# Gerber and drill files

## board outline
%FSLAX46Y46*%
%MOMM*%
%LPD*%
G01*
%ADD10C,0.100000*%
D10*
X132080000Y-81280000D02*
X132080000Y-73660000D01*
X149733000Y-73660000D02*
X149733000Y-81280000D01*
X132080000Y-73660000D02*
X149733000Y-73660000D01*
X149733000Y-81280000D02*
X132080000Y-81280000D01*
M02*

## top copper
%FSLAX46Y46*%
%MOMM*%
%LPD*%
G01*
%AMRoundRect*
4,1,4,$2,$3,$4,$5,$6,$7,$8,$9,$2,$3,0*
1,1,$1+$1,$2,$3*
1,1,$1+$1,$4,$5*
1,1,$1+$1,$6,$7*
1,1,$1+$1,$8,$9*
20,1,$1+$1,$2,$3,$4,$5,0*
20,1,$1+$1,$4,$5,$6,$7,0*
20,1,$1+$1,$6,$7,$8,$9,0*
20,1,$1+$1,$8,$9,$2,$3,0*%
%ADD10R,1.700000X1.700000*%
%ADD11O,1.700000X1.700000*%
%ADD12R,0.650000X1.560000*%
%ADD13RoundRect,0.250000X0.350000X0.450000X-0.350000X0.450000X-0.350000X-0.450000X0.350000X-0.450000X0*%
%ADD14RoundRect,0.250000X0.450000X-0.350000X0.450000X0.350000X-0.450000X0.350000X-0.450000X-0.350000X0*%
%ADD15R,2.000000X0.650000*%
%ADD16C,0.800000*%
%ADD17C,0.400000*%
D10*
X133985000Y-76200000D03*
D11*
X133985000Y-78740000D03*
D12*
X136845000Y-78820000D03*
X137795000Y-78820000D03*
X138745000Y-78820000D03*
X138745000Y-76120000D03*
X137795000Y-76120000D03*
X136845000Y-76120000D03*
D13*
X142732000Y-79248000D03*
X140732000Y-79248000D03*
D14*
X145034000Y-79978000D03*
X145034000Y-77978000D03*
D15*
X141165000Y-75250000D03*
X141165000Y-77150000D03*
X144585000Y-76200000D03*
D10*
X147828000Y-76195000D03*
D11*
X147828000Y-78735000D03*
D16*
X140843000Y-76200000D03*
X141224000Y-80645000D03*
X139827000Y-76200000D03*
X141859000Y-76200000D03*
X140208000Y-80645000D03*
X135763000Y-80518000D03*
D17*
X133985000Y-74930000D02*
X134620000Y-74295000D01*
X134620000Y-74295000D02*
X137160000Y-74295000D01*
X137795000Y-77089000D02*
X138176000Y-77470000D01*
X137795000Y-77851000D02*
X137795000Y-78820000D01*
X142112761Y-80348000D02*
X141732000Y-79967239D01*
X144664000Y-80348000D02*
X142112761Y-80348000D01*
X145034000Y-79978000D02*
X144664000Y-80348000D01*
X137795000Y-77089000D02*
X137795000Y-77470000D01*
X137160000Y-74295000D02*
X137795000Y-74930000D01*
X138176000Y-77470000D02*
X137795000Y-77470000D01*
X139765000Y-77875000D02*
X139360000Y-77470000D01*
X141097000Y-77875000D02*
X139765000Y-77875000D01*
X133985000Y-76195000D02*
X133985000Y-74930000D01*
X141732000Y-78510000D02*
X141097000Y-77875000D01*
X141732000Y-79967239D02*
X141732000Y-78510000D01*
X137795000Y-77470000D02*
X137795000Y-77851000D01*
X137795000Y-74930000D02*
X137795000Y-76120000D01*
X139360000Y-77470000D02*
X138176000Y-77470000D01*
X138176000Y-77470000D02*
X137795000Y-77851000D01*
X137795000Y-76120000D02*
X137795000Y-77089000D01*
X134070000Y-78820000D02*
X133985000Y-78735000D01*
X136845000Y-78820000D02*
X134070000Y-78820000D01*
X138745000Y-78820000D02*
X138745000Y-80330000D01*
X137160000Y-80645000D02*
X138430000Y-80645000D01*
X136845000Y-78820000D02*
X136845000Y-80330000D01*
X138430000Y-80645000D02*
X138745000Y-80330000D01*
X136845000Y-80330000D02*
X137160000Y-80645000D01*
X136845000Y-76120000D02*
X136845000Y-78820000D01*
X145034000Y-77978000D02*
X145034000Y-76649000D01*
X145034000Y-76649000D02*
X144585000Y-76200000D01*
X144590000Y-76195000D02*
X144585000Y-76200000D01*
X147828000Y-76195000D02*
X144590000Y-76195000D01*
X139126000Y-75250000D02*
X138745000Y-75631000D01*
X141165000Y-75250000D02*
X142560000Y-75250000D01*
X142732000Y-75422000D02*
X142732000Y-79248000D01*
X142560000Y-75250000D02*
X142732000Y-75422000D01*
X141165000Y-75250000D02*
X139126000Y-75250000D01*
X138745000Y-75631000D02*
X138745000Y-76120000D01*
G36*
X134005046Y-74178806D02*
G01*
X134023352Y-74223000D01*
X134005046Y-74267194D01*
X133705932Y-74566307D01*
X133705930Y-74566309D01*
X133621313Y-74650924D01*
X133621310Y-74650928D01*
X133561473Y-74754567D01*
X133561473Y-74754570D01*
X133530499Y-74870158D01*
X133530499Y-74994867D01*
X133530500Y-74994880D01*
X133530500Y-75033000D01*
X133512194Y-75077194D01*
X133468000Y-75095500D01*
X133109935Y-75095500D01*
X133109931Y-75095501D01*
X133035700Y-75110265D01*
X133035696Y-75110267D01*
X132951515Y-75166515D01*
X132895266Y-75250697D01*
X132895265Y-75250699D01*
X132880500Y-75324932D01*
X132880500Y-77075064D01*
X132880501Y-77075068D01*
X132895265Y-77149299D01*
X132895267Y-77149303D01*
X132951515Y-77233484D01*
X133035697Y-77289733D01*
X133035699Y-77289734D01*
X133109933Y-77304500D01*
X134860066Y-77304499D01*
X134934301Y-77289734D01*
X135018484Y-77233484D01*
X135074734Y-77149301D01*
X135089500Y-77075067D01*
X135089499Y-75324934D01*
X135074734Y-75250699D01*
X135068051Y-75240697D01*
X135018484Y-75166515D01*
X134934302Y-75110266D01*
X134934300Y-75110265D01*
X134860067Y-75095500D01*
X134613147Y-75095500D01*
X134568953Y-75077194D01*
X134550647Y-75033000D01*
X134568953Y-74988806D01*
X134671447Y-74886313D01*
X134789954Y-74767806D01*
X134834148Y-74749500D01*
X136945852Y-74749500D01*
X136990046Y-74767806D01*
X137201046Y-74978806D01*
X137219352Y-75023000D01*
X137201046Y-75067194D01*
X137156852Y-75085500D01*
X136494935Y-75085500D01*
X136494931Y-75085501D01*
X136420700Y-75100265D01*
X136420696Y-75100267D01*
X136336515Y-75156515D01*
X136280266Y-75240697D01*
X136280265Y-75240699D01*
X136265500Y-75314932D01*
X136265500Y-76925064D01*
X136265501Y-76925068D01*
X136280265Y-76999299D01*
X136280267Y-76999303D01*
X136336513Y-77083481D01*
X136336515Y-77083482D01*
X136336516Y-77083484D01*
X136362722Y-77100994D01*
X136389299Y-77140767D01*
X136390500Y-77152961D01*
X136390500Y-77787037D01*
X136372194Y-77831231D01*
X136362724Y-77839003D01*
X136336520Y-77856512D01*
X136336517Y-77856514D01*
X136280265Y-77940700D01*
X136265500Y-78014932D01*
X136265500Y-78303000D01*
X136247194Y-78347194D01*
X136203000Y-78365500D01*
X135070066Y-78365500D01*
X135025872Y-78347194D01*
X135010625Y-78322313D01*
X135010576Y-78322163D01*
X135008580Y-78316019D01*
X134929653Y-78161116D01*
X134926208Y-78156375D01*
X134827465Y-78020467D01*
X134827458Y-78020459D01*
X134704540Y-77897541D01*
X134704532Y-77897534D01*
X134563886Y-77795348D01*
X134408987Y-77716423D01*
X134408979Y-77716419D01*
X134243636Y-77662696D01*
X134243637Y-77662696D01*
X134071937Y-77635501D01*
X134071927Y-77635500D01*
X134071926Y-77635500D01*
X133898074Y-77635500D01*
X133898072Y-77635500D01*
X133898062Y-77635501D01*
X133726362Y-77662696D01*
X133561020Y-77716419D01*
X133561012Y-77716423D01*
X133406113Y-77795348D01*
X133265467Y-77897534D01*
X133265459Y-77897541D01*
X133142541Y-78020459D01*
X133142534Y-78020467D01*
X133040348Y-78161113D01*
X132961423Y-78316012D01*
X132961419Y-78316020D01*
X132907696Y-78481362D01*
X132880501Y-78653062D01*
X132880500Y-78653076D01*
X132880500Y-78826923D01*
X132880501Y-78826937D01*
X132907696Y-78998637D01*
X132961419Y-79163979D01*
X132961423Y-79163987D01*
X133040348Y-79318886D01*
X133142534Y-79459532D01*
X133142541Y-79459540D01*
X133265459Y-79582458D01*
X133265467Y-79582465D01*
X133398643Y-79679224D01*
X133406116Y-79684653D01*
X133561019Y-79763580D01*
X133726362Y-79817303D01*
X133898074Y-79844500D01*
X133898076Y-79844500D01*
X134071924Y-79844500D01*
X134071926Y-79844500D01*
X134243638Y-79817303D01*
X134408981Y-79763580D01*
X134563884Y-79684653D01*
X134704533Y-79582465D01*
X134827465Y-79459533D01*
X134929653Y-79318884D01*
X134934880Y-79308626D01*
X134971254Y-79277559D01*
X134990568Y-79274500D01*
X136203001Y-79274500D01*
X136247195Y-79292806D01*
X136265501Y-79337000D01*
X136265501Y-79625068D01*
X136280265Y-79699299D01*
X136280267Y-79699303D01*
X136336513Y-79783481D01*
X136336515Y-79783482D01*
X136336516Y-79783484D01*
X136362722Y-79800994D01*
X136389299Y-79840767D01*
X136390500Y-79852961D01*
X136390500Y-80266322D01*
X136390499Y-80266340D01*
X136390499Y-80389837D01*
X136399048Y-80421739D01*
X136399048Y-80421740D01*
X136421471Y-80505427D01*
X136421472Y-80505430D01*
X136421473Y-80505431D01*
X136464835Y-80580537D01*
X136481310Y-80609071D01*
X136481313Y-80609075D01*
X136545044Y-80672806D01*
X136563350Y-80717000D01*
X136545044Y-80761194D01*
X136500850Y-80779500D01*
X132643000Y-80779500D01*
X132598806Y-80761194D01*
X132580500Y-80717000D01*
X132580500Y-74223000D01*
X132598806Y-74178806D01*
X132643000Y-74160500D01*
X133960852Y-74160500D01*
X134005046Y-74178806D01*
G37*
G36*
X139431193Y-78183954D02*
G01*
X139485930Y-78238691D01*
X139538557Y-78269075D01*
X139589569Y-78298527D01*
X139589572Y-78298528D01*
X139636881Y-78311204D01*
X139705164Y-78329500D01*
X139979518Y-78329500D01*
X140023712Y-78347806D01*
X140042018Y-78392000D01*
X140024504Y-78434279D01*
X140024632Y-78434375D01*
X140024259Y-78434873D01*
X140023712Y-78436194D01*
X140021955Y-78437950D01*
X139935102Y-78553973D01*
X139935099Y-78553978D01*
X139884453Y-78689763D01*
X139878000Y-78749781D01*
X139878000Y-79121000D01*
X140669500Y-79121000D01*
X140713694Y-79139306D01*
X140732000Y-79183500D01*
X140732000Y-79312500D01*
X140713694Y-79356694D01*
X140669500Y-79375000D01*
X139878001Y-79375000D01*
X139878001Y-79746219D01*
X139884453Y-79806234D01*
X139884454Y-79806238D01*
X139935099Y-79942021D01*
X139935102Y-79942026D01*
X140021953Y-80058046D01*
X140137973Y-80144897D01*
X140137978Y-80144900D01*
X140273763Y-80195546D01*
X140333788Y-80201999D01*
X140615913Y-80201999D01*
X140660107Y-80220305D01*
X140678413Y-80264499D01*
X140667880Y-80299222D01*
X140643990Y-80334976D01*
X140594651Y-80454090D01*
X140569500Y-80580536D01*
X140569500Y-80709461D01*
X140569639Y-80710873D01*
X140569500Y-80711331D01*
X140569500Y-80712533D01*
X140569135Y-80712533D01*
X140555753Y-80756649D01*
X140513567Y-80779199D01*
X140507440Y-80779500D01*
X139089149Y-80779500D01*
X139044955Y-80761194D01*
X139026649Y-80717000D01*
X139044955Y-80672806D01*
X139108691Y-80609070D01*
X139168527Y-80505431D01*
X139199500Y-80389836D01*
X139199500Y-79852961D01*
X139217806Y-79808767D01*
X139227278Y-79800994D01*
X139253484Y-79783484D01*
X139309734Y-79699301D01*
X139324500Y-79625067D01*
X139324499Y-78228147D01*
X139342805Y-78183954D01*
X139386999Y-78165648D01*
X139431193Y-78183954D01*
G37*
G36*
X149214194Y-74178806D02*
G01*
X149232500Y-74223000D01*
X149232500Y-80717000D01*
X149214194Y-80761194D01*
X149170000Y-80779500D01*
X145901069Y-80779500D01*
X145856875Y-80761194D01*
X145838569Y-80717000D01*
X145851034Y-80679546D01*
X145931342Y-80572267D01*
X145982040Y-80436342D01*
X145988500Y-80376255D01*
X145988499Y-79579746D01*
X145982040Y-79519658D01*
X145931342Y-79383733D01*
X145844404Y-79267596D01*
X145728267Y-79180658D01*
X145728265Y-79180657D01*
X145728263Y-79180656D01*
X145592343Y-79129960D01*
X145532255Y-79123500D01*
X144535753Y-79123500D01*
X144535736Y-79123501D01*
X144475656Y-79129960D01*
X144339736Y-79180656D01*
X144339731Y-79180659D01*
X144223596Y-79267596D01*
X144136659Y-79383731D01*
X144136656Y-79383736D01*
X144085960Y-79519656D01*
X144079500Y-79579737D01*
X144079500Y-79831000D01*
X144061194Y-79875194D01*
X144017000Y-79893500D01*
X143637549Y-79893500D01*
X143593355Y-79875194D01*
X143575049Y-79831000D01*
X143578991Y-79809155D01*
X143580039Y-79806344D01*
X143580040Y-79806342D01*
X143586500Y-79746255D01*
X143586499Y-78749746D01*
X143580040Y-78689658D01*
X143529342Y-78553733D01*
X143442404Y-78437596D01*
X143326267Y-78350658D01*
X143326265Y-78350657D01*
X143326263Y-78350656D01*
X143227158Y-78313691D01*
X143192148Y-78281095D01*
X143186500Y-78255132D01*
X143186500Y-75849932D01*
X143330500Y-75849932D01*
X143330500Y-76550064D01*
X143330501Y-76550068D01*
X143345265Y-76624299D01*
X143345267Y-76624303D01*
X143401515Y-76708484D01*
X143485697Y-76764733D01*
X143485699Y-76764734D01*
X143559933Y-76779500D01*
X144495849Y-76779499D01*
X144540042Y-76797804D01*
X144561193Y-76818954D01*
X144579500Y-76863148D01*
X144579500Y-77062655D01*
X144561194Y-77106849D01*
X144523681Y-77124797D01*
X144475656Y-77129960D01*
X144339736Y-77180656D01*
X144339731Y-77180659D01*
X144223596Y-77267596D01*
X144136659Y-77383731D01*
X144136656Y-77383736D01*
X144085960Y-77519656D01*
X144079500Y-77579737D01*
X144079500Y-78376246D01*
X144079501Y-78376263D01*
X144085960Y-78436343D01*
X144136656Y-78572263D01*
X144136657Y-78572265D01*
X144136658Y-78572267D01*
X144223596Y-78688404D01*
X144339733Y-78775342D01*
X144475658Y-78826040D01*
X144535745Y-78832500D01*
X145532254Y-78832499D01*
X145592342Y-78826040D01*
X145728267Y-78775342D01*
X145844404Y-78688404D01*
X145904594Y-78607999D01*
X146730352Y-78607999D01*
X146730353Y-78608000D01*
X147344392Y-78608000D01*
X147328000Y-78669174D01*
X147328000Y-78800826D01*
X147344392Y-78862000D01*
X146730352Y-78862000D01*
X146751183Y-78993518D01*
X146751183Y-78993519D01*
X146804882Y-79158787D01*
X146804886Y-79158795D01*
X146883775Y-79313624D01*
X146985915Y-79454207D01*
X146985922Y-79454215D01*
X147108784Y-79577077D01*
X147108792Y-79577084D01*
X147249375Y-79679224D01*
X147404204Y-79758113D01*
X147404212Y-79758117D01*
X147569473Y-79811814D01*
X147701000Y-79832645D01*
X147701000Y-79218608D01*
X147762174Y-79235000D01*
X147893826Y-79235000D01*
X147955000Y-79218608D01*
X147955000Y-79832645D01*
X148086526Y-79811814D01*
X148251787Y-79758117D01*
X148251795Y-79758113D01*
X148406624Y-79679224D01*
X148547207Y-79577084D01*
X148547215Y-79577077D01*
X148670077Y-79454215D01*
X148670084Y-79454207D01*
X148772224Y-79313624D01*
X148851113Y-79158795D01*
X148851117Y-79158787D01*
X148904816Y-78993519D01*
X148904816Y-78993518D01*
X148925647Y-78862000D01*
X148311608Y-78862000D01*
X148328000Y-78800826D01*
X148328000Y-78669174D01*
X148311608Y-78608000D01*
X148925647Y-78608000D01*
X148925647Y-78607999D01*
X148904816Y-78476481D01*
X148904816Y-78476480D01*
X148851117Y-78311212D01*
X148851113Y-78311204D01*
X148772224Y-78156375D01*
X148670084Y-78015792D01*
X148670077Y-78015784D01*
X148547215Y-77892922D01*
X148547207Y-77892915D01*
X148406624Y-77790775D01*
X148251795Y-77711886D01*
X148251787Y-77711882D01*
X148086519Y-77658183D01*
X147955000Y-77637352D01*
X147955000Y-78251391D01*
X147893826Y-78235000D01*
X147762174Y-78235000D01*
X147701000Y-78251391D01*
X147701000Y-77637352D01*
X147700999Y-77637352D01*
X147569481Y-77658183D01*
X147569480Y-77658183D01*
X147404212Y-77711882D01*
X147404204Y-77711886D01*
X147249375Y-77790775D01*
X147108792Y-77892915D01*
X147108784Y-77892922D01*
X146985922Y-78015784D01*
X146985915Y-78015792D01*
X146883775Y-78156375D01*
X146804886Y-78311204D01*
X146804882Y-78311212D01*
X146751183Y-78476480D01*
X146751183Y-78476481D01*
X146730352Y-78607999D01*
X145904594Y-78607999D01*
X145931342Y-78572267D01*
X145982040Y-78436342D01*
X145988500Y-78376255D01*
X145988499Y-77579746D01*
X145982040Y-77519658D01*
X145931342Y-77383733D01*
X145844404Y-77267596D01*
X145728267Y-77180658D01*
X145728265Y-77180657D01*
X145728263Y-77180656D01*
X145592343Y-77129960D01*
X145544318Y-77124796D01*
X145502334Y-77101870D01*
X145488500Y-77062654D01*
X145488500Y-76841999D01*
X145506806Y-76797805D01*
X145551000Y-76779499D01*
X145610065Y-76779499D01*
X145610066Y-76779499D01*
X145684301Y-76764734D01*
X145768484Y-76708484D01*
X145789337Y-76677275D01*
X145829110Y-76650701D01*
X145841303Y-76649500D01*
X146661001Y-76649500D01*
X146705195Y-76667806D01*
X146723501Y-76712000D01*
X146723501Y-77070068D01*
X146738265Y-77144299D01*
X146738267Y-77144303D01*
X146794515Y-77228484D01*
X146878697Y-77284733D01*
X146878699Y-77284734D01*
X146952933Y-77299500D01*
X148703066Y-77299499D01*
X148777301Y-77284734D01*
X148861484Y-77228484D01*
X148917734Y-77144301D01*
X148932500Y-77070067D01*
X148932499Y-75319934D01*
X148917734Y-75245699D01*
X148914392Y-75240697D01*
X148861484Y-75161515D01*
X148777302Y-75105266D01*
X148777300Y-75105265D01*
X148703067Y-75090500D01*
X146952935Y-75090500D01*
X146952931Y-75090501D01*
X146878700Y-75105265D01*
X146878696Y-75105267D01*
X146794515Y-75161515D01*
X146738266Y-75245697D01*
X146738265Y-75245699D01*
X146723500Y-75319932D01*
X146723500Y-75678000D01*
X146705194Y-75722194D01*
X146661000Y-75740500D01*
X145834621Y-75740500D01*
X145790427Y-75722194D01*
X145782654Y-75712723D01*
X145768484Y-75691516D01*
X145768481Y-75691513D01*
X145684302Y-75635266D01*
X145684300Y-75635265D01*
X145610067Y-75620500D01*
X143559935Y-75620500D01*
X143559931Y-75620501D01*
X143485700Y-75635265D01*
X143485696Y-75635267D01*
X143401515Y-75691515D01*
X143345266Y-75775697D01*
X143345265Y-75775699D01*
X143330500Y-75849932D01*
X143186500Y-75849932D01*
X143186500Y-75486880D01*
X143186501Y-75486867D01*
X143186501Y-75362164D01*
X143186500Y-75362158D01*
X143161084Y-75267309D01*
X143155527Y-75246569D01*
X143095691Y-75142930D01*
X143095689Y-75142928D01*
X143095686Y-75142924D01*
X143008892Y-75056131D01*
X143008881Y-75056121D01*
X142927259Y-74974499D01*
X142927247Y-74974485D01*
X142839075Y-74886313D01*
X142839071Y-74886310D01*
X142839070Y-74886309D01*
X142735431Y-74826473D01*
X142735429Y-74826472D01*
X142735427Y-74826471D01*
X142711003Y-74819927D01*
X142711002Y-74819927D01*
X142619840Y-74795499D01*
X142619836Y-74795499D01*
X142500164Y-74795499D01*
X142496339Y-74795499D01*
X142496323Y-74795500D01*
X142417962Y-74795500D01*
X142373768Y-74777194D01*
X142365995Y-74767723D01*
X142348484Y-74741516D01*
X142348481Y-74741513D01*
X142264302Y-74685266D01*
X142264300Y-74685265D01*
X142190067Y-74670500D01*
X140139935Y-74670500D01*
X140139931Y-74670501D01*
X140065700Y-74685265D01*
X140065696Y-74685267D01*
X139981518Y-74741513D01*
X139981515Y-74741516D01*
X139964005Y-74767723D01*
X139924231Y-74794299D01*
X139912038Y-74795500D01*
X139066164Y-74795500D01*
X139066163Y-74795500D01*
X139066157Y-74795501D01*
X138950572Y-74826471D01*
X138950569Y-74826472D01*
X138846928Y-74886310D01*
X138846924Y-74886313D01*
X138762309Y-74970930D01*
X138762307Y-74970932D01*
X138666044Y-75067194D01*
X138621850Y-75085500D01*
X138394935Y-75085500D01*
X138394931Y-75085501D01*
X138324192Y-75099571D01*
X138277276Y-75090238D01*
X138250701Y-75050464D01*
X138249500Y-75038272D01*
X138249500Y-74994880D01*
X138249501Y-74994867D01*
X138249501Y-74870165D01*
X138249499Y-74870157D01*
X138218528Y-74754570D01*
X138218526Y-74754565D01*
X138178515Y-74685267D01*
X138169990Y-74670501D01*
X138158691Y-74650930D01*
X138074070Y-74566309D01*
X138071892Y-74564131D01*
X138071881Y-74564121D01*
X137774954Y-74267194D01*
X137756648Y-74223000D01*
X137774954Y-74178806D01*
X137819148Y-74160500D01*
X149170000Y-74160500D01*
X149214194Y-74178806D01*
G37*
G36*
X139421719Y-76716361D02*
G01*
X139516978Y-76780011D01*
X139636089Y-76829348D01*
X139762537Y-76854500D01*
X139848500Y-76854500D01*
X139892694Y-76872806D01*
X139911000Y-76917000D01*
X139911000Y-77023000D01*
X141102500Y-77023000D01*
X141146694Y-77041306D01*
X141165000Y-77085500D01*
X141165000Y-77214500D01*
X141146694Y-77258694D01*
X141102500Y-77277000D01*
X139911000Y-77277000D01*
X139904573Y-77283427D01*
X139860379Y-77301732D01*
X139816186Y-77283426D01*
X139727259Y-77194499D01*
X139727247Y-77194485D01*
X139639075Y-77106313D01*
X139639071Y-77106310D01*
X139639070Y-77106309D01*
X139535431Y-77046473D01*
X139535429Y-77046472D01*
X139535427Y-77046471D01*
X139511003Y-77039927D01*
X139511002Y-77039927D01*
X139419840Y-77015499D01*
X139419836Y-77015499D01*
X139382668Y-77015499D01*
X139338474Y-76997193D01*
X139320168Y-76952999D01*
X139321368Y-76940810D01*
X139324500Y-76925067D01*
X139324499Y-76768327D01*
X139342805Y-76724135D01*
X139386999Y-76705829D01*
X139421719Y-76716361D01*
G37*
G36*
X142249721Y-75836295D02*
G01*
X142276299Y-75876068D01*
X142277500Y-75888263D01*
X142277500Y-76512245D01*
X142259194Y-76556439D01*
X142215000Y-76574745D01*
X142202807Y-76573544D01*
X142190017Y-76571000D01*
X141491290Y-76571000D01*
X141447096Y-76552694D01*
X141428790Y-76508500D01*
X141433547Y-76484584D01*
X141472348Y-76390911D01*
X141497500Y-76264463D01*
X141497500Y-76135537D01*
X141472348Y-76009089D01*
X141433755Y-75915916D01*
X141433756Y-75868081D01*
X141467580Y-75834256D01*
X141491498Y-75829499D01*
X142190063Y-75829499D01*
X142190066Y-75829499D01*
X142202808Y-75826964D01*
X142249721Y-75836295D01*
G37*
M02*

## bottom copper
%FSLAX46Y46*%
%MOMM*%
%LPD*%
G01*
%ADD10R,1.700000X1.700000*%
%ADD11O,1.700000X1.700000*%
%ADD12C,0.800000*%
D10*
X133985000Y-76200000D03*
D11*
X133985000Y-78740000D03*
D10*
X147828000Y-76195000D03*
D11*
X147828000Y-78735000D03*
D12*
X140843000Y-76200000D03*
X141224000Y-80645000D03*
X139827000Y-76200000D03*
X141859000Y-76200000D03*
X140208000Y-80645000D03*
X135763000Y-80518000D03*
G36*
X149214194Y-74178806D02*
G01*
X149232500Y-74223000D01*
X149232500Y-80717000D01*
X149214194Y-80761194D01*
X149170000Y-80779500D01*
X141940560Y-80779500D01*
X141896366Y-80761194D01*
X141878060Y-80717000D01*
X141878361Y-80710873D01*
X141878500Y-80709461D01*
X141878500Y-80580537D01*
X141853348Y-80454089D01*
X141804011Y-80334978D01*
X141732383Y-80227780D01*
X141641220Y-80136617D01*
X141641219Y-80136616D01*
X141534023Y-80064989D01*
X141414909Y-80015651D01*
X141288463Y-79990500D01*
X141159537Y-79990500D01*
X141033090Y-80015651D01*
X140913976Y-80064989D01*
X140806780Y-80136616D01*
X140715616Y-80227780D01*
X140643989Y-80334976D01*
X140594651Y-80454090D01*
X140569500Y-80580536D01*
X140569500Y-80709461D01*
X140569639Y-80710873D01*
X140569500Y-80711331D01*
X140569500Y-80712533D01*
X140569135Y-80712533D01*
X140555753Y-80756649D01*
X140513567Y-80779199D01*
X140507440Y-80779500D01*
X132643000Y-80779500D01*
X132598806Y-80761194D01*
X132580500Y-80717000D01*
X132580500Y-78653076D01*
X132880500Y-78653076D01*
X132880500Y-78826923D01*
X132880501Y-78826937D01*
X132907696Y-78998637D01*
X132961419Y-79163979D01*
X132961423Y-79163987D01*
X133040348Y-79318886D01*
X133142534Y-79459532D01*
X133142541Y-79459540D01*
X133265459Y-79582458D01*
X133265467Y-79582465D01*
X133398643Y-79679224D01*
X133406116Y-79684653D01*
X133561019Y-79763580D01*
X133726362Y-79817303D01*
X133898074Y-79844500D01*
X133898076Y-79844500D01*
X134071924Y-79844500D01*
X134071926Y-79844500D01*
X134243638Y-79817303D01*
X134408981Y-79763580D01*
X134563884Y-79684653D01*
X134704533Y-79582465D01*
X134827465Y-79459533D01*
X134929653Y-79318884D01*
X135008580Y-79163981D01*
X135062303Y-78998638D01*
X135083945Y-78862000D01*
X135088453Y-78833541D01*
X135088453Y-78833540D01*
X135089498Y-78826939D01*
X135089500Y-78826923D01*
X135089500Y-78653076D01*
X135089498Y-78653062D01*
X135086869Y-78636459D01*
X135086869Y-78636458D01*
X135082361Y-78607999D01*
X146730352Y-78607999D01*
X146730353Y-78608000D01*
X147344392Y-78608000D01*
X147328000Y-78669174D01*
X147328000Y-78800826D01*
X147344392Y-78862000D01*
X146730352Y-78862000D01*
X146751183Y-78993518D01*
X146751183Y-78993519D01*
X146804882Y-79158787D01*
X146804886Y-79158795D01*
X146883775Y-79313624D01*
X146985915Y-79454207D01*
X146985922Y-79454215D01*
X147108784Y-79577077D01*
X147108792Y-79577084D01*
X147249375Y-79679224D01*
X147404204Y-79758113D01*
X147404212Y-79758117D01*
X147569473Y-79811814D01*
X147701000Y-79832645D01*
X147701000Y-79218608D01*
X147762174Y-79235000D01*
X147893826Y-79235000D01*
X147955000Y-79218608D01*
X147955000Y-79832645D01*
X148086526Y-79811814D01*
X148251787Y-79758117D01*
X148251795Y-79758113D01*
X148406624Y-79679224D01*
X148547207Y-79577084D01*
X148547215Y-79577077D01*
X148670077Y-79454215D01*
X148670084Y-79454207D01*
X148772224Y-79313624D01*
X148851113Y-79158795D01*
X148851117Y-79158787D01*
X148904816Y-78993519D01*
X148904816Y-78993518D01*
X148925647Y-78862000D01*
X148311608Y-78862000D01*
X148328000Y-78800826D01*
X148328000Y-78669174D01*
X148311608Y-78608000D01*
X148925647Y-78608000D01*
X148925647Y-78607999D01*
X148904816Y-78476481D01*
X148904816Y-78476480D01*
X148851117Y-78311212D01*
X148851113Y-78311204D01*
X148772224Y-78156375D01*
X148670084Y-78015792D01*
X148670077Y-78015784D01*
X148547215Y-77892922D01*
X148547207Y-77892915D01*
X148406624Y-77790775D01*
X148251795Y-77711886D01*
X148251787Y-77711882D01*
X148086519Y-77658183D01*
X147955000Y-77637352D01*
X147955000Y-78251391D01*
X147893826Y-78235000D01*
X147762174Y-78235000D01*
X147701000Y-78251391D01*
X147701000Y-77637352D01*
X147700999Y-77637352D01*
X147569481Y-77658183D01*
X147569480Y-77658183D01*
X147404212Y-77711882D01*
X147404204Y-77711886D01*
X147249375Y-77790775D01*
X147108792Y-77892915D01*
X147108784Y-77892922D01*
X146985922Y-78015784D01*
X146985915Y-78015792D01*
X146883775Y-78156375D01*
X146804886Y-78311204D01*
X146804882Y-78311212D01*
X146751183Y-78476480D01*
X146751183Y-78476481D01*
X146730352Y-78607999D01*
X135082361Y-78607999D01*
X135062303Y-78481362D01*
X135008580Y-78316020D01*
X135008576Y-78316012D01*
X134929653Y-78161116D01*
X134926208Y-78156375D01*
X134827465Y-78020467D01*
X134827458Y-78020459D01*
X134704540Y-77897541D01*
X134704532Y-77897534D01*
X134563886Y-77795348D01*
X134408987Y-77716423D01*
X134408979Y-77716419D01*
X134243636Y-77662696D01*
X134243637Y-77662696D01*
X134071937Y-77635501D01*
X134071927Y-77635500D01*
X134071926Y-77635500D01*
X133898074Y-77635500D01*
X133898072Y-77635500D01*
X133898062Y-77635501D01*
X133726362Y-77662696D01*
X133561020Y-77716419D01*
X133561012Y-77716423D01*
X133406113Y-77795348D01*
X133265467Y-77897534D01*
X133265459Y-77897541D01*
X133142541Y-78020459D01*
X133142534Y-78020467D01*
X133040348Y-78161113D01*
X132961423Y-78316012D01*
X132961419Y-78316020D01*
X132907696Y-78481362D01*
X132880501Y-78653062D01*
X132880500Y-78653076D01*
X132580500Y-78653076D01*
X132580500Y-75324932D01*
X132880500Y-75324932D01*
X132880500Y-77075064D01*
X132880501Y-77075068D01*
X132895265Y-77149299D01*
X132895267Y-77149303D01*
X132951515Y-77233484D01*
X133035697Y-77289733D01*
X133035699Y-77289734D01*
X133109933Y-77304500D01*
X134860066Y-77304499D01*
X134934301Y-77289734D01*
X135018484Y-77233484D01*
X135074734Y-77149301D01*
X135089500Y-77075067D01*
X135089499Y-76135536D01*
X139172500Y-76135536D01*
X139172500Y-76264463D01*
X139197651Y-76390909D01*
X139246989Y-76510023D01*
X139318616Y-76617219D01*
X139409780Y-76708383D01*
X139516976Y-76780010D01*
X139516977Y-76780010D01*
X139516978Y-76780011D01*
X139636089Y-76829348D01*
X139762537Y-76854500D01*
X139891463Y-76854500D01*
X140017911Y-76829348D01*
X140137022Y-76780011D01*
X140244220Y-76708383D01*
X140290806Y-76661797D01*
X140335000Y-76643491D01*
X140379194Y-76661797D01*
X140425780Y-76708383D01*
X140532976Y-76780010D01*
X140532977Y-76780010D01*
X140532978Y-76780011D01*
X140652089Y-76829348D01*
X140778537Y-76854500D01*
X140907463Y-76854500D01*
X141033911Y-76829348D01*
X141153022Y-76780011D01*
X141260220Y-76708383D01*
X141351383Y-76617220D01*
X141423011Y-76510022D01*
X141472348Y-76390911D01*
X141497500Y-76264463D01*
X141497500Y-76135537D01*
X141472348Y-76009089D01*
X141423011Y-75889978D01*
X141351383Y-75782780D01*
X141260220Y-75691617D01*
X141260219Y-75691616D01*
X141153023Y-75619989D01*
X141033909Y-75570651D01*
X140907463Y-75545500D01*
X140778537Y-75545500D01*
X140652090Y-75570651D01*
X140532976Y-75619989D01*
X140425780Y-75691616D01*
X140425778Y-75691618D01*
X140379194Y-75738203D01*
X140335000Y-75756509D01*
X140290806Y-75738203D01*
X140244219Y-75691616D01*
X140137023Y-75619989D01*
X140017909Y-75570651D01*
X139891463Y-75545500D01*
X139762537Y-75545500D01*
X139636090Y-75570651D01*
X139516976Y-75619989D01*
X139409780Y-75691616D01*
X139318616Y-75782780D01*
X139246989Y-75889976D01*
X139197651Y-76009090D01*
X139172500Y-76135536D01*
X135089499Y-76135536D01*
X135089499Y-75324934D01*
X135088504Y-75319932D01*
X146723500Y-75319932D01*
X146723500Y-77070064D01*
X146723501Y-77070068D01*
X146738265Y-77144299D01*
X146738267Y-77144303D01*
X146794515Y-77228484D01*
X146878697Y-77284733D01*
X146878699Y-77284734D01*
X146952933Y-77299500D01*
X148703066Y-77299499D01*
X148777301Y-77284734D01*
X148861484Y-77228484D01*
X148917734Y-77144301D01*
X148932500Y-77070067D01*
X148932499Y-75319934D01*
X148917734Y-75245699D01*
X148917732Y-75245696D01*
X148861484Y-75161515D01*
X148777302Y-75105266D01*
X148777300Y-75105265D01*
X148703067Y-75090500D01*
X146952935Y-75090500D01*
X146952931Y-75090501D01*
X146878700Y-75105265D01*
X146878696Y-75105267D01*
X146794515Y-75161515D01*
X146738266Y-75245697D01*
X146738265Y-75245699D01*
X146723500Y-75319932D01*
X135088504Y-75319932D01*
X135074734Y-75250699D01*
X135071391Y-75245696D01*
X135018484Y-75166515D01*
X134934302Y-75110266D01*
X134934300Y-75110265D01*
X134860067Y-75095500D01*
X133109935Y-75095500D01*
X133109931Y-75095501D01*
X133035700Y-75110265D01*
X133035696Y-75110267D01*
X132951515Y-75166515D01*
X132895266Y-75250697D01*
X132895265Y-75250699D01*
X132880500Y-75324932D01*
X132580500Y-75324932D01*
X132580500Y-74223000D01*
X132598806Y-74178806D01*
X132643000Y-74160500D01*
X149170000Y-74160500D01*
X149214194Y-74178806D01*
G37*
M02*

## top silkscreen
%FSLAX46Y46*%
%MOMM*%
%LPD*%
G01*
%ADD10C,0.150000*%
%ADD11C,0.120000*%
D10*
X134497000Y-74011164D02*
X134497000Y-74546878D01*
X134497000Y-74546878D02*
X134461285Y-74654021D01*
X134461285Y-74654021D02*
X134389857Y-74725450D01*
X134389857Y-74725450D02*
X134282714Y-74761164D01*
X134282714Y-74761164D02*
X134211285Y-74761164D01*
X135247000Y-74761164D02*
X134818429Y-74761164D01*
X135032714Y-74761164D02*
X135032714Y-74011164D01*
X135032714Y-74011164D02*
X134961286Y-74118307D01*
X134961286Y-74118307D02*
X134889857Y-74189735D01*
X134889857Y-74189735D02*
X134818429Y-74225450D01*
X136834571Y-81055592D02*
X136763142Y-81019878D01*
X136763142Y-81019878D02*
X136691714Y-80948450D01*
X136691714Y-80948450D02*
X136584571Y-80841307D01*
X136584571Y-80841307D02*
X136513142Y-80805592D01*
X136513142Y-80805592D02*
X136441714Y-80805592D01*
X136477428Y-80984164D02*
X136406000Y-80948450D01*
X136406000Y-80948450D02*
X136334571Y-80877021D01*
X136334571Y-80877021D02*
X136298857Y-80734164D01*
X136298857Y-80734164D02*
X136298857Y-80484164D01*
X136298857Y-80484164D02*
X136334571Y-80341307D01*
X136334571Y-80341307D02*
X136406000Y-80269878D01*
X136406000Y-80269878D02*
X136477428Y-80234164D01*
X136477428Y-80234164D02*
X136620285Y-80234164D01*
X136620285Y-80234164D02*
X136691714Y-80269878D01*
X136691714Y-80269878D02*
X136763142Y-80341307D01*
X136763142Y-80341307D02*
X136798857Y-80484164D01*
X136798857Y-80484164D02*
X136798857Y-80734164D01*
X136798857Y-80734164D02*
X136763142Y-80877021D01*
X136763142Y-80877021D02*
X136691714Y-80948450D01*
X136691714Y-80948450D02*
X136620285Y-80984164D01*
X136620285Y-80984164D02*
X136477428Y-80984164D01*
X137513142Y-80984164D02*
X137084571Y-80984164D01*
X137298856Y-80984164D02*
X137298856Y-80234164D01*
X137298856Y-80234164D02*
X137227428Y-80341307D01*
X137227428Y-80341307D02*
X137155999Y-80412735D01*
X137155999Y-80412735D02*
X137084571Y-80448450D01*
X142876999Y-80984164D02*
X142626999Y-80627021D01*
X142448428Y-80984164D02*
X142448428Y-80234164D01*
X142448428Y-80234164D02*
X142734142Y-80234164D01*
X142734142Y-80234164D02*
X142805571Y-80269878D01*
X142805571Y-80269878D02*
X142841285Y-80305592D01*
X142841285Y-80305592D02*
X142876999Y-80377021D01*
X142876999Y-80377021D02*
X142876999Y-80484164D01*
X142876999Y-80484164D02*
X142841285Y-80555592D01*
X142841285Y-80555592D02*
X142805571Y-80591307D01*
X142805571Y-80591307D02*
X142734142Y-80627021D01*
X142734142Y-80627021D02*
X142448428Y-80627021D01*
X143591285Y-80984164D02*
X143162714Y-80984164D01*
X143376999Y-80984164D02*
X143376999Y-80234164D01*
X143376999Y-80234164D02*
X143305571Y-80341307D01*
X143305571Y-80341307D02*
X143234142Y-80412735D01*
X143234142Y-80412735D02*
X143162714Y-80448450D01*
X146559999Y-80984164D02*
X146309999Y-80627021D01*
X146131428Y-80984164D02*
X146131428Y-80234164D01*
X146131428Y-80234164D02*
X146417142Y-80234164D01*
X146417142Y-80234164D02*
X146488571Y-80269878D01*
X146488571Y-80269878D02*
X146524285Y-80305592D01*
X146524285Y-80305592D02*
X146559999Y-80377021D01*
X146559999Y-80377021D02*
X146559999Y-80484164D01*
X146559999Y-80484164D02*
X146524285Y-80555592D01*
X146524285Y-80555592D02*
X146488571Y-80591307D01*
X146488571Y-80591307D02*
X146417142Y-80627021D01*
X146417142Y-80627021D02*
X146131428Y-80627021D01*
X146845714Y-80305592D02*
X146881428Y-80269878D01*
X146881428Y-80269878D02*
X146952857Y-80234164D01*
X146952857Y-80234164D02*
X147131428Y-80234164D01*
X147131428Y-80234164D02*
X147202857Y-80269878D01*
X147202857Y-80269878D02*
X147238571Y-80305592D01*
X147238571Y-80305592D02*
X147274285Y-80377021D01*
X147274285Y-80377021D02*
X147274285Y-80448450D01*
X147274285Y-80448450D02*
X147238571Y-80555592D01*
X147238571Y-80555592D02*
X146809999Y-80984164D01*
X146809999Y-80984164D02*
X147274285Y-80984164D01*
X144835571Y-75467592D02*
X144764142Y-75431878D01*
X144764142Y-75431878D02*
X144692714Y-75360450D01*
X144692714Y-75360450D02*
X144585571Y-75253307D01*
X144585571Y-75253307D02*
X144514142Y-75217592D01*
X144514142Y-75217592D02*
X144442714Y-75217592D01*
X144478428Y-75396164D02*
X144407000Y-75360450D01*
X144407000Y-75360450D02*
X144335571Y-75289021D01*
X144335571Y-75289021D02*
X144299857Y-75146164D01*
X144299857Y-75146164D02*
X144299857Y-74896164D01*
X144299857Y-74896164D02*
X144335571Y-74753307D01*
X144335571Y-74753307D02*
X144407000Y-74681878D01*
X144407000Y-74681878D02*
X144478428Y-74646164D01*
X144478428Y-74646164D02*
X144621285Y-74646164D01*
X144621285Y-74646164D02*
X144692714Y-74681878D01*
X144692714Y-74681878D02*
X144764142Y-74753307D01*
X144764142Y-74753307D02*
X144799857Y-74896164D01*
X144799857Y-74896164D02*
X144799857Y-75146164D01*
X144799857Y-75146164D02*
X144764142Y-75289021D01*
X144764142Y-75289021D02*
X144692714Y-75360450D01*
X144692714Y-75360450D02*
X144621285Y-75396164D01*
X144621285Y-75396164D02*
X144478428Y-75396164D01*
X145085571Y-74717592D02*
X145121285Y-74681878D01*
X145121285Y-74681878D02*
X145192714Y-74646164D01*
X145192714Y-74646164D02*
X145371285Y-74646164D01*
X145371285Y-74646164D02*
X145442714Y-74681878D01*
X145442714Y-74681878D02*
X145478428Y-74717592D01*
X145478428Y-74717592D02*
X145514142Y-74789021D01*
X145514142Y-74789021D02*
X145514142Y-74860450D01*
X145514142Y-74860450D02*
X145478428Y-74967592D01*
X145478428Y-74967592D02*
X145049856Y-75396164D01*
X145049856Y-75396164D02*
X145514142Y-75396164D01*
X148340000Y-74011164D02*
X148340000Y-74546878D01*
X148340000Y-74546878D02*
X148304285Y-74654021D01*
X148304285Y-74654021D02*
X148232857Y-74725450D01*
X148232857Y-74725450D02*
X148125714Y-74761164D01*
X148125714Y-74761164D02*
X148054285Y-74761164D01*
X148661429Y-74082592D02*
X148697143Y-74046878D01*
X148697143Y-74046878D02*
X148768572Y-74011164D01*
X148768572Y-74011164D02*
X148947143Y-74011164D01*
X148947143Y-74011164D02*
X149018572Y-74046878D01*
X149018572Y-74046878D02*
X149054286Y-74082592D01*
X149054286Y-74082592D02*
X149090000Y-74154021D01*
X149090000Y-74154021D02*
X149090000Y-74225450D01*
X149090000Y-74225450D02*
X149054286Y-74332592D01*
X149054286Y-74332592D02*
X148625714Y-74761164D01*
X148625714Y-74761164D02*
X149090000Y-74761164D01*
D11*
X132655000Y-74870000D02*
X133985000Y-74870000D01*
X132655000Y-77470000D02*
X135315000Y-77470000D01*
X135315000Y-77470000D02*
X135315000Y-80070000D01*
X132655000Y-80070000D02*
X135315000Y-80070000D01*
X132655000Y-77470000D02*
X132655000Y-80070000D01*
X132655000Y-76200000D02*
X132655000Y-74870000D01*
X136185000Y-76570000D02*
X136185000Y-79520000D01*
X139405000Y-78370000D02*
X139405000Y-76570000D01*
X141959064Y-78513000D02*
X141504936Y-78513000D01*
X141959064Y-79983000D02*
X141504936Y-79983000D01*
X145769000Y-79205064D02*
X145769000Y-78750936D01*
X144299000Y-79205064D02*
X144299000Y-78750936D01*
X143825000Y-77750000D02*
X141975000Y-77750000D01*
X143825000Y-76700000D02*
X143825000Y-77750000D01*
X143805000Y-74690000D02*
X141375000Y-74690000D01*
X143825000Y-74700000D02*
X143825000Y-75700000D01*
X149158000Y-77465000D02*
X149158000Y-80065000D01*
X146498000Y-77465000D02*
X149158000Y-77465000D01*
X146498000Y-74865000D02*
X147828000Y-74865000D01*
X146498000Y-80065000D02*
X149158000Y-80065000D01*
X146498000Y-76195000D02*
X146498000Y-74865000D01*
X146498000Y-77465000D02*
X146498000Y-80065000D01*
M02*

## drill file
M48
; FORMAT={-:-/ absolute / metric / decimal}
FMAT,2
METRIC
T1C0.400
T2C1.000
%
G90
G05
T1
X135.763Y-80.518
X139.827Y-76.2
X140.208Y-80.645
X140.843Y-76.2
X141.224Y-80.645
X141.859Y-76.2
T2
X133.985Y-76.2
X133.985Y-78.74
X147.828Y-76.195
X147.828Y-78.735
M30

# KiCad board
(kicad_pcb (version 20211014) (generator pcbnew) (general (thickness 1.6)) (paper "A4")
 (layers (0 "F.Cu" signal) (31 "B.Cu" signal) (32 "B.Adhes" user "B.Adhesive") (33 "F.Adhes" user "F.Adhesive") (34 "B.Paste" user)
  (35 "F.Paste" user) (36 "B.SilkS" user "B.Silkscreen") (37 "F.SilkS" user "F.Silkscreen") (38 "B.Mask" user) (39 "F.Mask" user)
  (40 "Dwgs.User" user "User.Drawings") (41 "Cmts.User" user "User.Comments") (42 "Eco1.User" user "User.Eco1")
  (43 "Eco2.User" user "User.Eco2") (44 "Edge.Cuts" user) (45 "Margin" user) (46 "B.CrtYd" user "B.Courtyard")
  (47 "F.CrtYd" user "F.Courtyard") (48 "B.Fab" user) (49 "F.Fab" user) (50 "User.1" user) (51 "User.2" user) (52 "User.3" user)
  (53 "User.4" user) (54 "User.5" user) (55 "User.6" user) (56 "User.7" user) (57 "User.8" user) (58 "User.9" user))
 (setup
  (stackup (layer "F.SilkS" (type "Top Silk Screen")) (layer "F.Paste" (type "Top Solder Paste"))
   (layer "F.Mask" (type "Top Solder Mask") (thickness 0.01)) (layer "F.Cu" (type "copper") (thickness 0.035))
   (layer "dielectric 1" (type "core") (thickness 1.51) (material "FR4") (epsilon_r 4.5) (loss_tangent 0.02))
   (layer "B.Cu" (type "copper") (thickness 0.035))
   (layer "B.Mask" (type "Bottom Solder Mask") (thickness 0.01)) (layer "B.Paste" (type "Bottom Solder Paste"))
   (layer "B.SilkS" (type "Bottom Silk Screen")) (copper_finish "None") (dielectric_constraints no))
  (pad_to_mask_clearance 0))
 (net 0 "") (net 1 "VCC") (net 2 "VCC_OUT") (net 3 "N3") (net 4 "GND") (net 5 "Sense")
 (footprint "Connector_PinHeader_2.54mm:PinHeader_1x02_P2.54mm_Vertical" (layer "F.Cu") (at 133.985 76.2)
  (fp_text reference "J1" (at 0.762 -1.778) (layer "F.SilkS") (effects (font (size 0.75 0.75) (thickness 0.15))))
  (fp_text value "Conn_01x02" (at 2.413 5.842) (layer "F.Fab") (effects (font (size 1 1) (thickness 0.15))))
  (fp_line (start -1.33 -1.33) (end 0 -1.33) (layer "F.SilkS") (width 0.12))
  (fp_line (start -1.33 1.27) (end 1.33 1.27) (layer "F.SilkS") (width 0.12))
  (fp_line (start 1.33 1.27) (end 1.33 3.87) (layer "F.SilkS") (width 0.12))
  (fp_line (start -1.33 3.87) (end 1.33 3.87) (layer "F.SilkS") (width 0.12))
  (fp_line (start -1.33 1.27) (end -1.33 3.87) (layer "F.SilkS") (width 0.12))
  (fp_line (start -1.33 0) (end -1.33 -1.33) (layer "F.SilkS") (width 0.12))
  (pad "1" thru_hole rect (at 0 0) (size 1.7 1.7) (drill 1) (layers *.Cu *.Mask) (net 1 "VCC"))
  (pad "2" thru_hole oval (at 0 2.54) (size 1.7 1.7) (drill 1) (layers *.Cu *.Mask) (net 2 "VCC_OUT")))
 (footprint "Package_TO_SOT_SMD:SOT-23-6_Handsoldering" (layer "F.Cu") (at 137.795 77.47 90)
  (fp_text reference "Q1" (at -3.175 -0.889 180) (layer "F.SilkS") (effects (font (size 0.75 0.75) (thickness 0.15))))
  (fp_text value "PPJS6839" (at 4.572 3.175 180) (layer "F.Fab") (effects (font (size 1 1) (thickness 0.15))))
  (fp_line (start 0.9 -1.61) (end -2.05 -1.61) (layer "F.SilkS") (width 0.12))
  (fp_line (start -0.9 1.61) (end 0.9 1.61) (layer "F.SilkS") (width 0.12))
  (pad "1" smd rect (at -1.35 -0.95 90) (size 1.56 0.65) (layers "F.Cu" "F.Paste" "F.Mask") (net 2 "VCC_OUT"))
  (pad "2" smd rect (at -1.35 0 90) (size 1.56 0.65) (layers "F.Cu" "F.Paste" "F.Mask") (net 1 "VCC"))
  (pad "3" smd rect (at -1.35 0.95 90) (size 1.56 0.65) (layers "F.Cu" "F.Paste" "F.Mask") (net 2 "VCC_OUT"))
  (pad "4" smd rect (at 1.35 0.95 90) (size 1.56 0.65) (layers "F.Cu" "F.Paste" "F.Mask") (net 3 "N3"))
  (pad "5" smd rect (at 1.35 0 90) (size 1.56 0.65) (layers "F.Cu" "F.Paste" "F.Mask") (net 1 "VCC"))
  (pad "6" smd rect (at 1.35 -0.95 90) (size 1.56 0.65) (layers "F.Cu" "F.Paste" "F.Mask") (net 2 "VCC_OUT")))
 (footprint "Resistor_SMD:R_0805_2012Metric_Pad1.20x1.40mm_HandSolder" (layer "F.Cu") (at 141.732 79.248 180)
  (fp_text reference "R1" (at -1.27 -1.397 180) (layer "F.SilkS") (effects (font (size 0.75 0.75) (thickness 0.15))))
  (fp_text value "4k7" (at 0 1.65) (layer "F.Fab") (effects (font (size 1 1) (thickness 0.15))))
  (fp_line (start -0.227064 0.735) (end 0.227064 0.735) (layer "F.SilkS") (width 0.12))
  (fp_line (start -0.227064 -0.735) (end 0.227064 -0.735) (layer "F.SilkS") (width 0.12))
  (pad "1" smd roundrect (at -1 0 180) (size 1.2 1.4) (layers "F.Cu" "F.Paste" "F.Mask") (roundrect_rratio 0.208333) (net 3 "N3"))
  (pad "2" smd roundrect (at 1 0 180) (size 1.2 1.4) (layers "F.Cu" "F.Paste" "F.Mask") (roundrect_rratio 0.208333) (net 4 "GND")))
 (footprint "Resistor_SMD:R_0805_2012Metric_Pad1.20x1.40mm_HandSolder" (layer "F.Cu") (at 145.034 78.978 90)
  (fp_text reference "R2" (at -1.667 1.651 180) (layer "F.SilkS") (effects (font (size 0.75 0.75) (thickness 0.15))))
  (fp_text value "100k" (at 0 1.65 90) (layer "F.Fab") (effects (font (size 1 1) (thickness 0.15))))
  (fp_line (start -0.227064 0.735) (end 0.227064 0.735) (layer "F.SilkS") (width 0.12))
  (fp_line (start -0.227064 -0.735) (end 0.227064 -0.735) (layer "F.SilkS") (width 0.12))
  (pad "1" smd roundrect (at -1 0 90) (size 1.2 1.4) (layers "F.Cu" "F.Paste" "F.Mask") (roundrect_rratio 0.208333) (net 1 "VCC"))
  (pad "2" smd roundrect (at 1 0 90) (size 1.2 1.4) (layers "F.Cu" "F.Paste" "F.Mask") (roundrect_rratio 0.208333) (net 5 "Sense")))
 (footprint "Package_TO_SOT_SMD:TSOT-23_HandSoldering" (layer "F.Cu") (at 142.875 76.2)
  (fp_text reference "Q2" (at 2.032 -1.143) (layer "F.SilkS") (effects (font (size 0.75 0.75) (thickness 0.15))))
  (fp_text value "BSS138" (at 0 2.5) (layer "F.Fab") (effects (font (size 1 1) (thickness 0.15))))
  (fp_line (start 0.95 1.55) (end -0.9 1.55) (layer "F.SilkS") (width 0.12))
  (fp_line (start 0.95 0.5) (end 0.95 1.55) (layer "F.SilkS") (width 0.12))
  (fp_line (start 0.93 -1.51) (end -1.5 -1.51) (layer "F.SilkS") (width 0.12))
  (fp_line (start 0.95 -1.5) (end 0.95 -0.5) (layer "F.SilkS") (width 0.12))
  (pad "1" smd rect (at -1.71 -0.95) (size 2 0.65) (layers "F.Cu" "F.Paste" "F.Mask") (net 3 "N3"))
  (pad "2" smd rect (at -1.71 0.95) (size 2 0.65) (layers "F.Cu" "F.Paste" "F.Mask") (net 4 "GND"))
  (pad "3" smd rect (at 1.71 0) (size 2 0.65) (layers "F.Cu" "F.Paste" "F.Mask") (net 5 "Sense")))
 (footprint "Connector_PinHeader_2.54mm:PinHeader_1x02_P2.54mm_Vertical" (layer "F.Cu") (at 147.828 76.195)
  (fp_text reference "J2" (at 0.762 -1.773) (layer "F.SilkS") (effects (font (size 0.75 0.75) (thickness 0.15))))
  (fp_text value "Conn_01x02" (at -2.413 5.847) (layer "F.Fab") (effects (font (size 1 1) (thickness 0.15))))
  (fp_line (start 1.33 1.27) (end 1.33 3.87) (layer "F.SilkS") (width 0.12))
  (fp_line (start -1.33 1.27) (end 1.33 1.27) (layer "F.SilkS") (width 0.12))
  (fp_line (start -1.33 -1.33) (end 0 -1.33) (layer "F.SilkS") (width 0.12))
  (fp_line (start -1.33 3.87) (end 1.33 3.87) (layer "F.SilkS") (width 0.12))
  (fp_line (start -1.33 0) (end -1.33 -1.33) (layer "F.SilkS") (width 0.12))
  (fp_line (start -1.33 1.27) (end -1.33 3.87) (layer "F.SilkS") (width 0.12))
  (pad "1" thru_hole rect (at 0 0) (size 1.7 1.7) (drill 1) (layers *.Cu *.Mask) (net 5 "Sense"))
  (pad "2" thru_hole oval (at 0 2.54) (size 1.7 1.7) (drill 1) (layers *.Cu *.Mask) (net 4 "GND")))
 (gr_line (start 132.08 81.28) (end 132.08 73.66) (layer "Edge.Cuts") (width 0.1))
 (gr_line (start 149.733 73.66) (end 149.733 81.28) (layer "Edge.Cuts") (width 0.1))
 (gr_line (start 132.08 73.66) (end 149.733 73.66) (layer "Edge.Cuts") (width 0.1))
 (gr_line (start 149.733 81.28) (end 132.08 81.28) (layer "Edge.Cuts") (width 0.1))
 (via (at 140.843 76.2) (size 0.8) (drill 0.4) (layers "F.Cu" "B.Cu") (free) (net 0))
 (via (at 141.224 80.645) (size 0.8) (drill 0.4) (layers "F.Cu" "B.Cu") (free) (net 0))
 (via (at 139.827 76.2) (size 0.8) (drill 0.4) (layers "F.Cu" "B.Cu") (free) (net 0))
 (segment (start 133.985 74.93) (end 134.62 74.295) (width 0.4) (layer "F.Cu") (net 1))
 (segment (start 134.62 74.295) (end 137.16 74.295) (width 0.4) (layer "F.Cu") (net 1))
 (segment (start 137.795 77.089) (end 138.176 77.47) (width 0.4) (layer "F.Cu") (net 1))
 (segment (start 137.795 77.851) (end 137.795 78.82) (width 0.4) (layer "F.Cu") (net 1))
 (segment (start 142.112761 80.348) (end 141.732 79.967239) (width 0.4) (layer "F.Cu") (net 1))
 (segment (start 144.664 80.348) (end 142.112761 80.348) (width 0.4) (layer "F.Cu") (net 1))
 (segment (start 145.034 79.978) (end 144.664 80.348) (width 0.4) (layer "F.Cu") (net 1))
 (segment (start 137.795 77.089) (end 137.795 77.47) (width 0.4) (layer "F.Cu") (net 1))
 (segment (start 137.16 74.295) (end 137.795 74.93) (width 0.4) (layer "F.Cu") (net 1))
 (segment (start 138.176 77.47) (end 137.795 77.47) (width 0.4) (layer "F.Cu") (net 1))
 (segment (start 139.765 77.875) (end 139.36 77.47) (width 0.4) (layer "F.Cu") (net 1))
 (segment (start 141.097 77.875) (end 139.765 77.875) (width 0.4) (layer "F.Cu") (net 1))
 (segment (start 133.985 76.195) (end 133.985 74.93) (width 0.4) (layer "F.Cu") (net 1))
 (segment (start 141.732 78.51) (end 141.097 77.875) (width 0.4) (layer "F.Cu") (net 1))
 (segment (start 141.732 79.967239) (end 141.732 78.51) (width 0.4) (layer "F.Cu") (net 1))
 (segment (start 137.795 77.47) (end 137.795 77.851) (width 0.4) (layer "F.Cu") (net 1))
 (segment (start 137.795 74.93) (end 137.795 76.12) (width 0.4) (layer "F.Cu") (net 1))
 (segment (start 139.36 77.47) (end 138.176 77.47) (width 0.4) (layer "F.Cu") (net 1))
 (segment (start 138.176 77.47) (end 137.795 77.851) (width 0.4) (layer "F.Cu") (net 1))
 (segment (start 137.795 76.12) (end 137.795 77.089) (width 0.4) (layer "F.Cu") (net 1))
 (segment (start 134.07 78.82) (end 133.985 78.735) (width 0.4) (layer "F.Cu") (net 2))
 (segment (start 136.845 78.82) (end 134.07 78.82) (width 0.4) (layer "F.Cu") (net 2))
 (segment (start 138.745 78.82) (end 138.745 80.33) (width 0.4) (layer "F.Cu") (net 2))
 (segment (start 137.16 80.645) (end 138.43 80.645) (width 0.4) (layer "F.Cu") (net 2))
 (segment (start 136.845 78.82) (end 136.845 80.33) (width 0.4) (layer "F.Cu") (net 2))
 (segment (start 138.43 80.645) (end 138.745 80.33) (width 0.4) (layer "F.Cu") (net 2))
 (segment (start 136.845 80.33) (end 137.16 80.645) (width 0.4) (layer "F.Cu") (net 2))
 (segment (start 136.845 76.12) (end 136.845 78.82) (width 0.4) (layer "F.Cu") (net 2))
 (segment (start 145.034 77.978) (end 145.034 76.649) (width 0.4) (layer "F.Cu") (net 5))
 (segment (start 145.034 76.649) (end 144.585 76.2) (width 0.4) (layer "F.Cu") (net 5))
 (segment (start 144.59 76.195) (end 144.585 76.2) (width 0.4) (layer "F.Cu") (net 5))
 (segment (start 147.828 76.195) (end 144.59 76.195) (width 0.4) (layer "F.Cu") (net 5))
 (via (at 141.859 76.2) (size 0.8) (drill 0.4) (layers "F.Cu" "B.Cu") (free) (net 4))
 (via (at 140.208 80.645) (size 0.8) (drill 0.4) (layers "F.Cu" "B.Cu") (free) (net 4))
 (via (at 135.763 80.518) (size 0.8) (drill 0.4) (layers "F.Cu" "B.Cu") (free) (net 4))
 (segment (start 139.126 75.25) (end 138.745 75.631) (width 0.4) (layer "F.Cu") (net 3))
 (segment (start 141.165 75.25) (end 142.56 75.25) (width 0.4) (layer "F.Cu") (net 3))
 (segment (start 142.732 75.422) (end 142.732 79.248) (width 0.4) (layer "F.Cu") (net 3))
 (segment (start 142.56 75.25) (end 142.732 75.422) (width 0.4) (layer "F.Cu") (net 3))
 (segment (start 141.165 75.25) (end 139.126 75.25) (width 0.4) (layer "F.Cu") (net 3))
 (segment (start 138.745 75.631) (end 138.745 76.12) (width 0.4) (layer "F.Cu") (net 3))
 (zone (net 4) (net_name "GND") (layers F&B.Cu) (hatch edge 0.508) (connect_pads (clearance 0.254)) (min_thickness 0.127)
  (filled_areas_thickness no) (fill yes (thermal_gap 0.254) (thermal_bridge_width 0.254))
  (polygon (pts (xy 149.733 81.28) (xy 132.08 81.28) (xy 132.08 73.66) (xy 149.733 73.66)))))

